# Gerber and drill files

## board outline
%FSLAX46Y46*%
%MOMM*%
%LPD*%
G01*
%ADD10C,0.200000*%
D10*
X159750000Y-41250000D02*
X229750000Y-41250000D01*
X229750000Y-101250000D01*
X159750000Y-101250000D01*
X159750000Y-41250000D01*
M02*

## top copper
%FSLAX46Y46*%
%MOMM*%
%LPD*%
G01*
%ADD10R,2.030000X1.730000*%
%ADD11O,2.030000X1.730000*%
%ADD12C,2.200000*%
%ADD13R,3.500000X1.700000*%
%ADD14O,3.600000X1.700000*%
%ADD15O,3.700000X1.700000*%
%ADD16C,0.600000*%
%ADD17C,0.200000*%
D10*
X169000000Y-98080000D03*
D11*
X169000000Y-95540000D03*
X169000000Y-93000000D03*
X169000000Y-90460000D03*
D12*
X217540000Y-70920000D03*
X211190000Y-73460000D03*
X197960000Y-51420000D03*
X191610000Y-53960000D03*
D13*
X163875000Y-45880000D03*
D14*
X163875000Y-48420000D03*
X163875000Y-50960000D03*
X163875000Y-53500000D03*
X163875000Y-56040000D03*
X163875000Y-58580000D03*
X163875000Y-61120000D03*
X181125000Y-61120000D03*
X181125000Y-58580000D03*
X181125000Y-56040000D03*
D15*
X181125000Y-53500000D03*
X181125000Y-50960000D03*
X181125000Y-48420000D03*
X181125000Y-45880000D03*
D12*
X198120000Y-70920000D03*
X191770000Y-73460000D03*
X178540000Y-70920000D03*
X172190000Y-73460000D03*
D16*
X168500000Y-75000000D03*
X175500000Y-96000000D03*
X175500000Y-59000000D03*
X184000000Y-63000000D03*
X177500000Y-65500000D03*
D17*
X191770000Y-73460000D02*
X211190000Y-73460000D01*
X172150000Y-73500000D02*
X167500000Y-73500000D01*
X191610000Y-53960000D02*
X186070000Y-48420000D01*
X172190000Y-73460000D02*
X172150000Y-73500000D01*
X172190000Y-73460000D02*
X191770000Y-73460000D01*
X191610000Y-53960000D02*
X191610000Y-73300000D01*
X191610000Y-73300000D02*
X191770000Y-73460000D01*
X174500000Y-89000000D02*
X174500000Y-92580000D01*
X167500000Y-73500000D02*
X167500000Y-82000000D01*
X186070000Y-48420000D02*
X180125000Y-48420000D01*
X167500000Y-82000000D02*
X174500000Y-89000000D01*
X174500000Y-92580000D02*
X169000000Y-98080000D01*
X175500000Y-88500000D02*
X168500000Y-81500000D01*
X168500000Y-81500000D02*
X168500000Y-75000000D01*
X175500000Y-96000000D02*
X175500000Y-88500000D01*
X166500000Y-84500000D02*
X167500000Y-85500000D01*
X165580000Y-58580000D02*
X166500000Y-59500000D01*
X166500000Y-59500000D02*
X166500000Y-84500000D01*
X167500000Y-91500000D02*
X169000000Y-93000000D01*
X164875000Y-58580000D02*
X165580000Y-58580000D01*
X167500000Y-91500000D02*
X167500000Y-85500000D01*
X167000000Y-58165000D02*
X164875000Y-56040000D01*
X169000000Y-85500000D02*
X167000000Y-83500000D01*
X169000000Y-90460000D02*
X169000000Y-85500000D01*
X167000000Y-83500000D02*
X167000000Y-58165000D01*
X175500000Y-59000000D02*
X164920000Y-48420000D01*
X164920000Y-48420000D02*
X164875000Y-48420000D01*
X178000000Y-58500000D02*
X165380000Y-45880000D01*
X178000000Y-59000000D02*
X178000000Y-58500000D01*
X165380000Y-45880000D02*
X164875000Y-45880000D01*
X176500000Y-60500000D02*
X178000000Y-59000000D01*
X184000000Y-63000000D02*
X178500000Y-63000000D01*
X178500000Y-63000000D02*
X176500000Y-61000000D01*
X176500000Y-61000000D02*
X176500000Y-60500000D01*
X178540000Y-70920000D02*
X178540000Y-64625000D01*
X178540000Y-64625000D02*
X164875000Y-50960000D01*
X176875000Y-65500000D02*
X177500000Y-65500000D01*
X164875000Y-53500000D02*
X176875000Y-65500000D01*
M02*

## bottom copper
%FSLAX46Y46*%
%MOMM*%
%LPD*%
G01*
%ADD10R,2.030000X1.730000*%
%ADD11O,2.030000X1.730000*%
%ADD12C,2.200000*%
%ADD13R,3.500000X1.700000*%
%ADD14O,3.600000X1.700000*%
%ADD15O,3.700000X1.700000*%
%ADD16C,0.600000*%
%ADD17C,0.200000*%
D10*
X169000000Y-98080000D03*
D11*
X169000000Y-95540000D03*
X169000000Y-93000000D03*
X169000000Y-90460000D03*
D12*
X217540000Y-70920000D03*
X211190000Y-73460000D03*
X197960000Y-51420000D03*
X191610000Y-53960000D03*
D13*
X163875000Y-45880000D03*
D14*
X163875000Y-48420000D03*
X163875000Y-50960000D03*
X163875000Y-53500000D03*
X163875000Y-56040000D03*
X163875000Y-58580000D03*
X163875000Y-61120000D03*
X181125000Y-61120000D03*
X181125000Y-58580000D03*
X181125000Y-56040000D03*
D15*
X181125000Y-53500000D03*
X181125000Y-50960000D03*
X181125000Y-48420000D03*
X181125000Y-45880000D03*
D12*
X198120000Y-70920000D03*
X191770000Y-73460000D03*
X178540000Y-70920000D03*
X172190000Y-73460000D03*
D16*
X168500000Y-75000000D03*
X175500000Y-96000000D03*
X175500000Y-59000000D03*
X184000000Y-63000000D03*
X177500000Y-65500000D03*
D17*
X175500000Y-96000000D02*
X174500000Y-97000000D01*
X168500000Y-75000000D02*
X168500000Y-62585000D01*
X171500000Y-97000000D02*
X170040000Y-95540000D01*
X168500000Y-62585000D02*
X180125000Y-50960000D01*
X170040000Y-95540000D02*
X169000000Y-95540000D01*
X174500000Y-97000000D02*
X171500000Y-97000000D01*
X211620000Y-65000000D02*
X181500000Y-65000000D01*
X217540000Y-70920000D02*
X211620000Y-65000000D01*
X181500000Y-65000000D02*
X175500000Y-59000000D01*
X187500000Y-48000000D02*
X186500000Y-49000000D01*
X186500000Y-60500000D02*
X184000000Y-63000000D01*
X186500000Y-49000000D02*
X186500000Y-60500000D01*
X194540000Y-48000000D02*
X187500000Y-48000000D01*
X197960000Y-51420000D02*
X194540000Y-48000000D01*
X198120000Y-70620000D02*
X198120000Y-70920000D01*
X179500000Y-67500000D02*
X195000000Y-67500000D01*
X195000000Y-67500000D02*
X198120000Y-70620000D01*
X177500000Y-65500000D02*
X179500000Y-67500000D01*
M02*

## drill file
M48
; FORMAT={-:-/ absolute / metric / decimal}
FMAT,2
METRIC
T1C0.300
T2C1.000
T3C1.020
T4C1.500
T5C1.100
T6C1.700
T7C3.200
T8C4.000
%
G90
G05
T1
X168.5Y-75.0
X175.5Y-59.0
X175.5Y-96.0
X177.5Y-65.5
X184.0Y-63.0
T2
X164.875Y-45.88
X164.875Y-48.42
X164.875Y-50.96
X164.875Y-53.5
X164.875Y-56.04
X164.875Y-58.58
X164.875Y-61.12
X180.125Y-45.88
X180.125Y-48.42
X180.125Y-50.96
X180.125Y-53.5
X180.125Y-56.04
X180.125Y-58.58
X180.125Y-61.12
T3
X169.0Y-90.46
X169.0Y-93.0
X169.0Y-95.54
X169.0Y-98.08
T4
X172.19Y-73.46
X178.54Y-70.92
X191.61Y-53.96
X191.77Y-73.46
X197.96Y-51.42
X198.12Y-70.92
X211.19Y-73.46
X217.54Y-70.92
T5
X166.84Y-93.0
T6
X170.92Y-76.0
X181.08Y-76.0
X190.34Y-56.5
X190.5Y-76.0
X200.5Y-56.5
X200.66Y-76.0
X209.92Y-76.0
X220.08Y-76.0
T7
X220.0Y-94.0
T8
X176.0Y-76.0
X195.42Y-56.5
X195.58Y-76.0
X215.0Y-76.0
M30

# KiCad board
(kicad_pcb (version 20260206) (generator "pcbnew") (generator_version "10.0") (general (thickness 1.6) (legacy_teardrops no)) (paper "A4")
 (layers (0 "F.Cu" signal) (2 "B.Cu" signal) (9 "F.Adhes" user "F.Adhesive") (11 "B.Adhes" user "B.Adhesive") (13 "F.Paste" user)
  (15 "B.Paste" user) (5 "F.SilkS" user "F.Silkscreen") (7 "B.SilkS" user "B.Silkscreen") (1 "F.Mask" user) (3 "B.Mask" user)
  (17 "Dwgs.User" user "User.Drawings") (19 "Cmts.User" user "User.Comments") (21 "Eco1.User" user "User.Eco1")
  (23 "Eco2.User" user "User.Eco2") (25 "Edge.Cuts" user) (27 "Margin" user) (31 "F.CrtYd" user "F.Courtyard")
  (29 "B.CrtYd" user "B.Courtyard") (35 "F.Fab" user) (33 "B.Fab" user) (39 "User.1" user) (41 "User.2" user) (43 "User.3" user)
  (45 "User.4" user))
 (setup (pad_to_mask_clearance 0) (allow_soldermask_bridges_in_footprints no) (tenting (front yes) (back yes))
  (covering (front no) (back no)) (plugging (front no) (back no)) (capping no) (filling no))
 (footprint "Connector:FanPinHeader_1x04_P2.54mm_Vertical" (layer "F.Cu") (at 169 98.08 90)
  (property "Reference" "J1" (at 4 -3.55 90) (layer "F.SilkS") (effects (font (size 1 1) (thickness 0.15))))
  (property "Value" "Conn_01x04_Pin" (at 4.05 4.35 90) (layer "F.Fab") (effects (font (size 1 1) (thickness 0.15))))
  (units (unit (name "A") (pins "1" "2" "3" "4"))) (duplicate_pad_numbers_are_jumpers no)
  (pad "" np_thru_hole circle (at 5.08 -2.16 180) (size 1.1 1.1) (drill 1.1) (layers "*.Cu" "*.Mask"))
  (pad "1" thru_hole rect (at 0 0 180) (size 2.03 1.73) (drill 1.02) (layers "*.Cu" "*.Mask") (remove_unused_layers no)
   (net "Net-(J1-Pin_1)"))
  (pad "2" thru_hole oval (at 2.54 0 180) (size 2.03 1.73) (drill 1.02) (layers "*.Cu" "*.Mask") (remove_unused_layers no)
   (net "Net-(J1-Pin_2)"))
  (pad "3" thru_hole oval (at 5.08 0 180) (size 2.03 1.73) (drill 1.02) (layers "*.Cu" "*.Mask") (remove_unused_layers no)
   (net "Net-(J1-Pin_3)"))
  (pad "4" thru_hole oval (at 7.62 0 180) (size 2.03 1.73) (drill 1.02) (layers "*.Cu" "*.Mask") (remove_unused_layers no)
   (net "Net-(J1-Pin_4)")))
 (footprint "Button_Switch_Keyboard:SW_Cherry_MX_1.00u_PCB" (layer "F.Cu") (at 217.54 70.92)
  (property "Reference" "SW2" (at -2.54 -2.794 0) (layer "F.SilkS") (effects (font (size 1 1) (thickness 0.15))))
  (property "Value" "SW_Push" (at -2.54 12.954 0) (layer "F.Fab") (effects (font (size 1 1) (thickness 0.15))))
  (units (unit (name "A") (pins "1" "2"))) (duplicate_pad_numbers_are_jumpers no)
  (pad "" np_thru_hole circle (at -7.62 5.08) (size 1.7 1.7) (drill 1.7) (layers "*.Cu" "*.Mask"))
  (pad "" np_thru_hole circle (at -2.54 5.08) (size 4 4) (drill 4) (layers "*.Cu" "*.Mask"))
  (pad "" np_thru_hole circle (at 2.54 5.08) (size 1.7 1.7) (drill 1.7) (layers "*.Cu" "*.Mask"))
  (pad "1" thru_hole circle (at 0 0) (size 2.2 2.2) (drill 1.5) (layers "*.Cu" "*.Mask") (remove_unused_layers no)
   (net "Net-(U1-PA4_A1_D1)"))
  (pad "2" thru_hole circle (at -6.35 2.54) (size 2.2 2.2) (drill 1.5) (layers "*.Cu" "*.Mask") (remove_unused_layers no)
   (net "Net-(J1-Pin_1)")))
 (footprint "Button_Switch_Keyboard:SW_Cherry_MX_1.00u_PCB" (layer "F.Cu") (at 197.96 51.42)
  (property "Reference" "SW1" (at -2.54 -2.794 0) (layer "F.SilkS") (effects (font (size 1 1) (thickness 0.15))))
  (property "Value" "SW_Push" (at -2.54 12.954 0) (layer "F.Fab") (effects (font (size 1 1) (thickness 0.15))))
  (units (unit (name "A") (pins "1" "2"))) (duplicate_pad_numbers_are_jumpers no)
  (pad "" np_thru_hole circle (at -7.62 5.08) (size 1.7 1.7) (drill 1.7) (layers "*.Cu" "*.Mask"))
  (pad "" np_thru_hole circle (at -2.54 5.08) (size 4 4) (drill 4) (layers "*.Cu" "*.Mask"))
  (pad "" np_thru_hole circle (at 2.54 5.08) (size 1.7 1.7) (drill 1.7) (layers "*.Cu" "*.Mask"))
  (pad "1" thru_hole circle (at 0 0) (size 2.2 2.2) (drill 1.5) (layers "*.Cu" "*.Mask") (remove_unused_layers no)
   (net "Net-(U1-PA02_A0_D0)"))
  (pad "2" thru_hole circle (at -6.35 2.54) (size 2.2 2.2) (drill 1.5) (layers "*.Cu" "*.Mask") (remove_unused_layers no)
   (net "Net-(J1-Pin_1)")))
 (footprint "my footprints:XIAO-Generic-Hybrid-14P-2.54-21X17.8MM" (layer "F.Cu") (at 172.5 53.5)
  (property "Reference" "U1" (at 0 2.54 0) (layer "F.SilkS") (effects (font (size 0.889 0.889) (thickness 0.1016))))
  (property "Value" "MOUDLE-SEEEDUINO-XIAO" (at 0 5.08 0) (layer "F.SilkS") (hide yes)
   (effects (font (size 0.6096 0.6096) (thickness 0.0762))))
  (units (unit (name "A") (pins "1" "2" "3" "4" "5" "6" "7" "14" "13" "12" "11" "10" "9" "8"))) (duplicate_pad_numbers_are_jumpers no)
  (pad "1" thru_hole rect (at -7.625 -7.62) (size 3.5 1.7) (drill 1 (offset -1 0)) (layers "*.Cu" "*.Mask") (remove_unused_layers no)
   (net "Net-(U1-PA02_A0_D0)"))
  (pad "2" thru_hole oval (at -7.625 -5.08) (size 3.6 1.7) (drill 1 (offset -1 0)) (layers "*.Cu" "*.Mask") (remove_unused_layers no)
   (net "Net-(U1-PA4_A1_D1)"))
  (pad "3" thru_hole oval (at -7.625 -2.54) (size 3.6 1.7) (drill 1 (offset -1 0)) (layers "*.Cu" "*.Mask") (remove_unused_layers no)
   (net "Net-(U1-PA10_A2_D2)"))
  (pad "4" thru_hole oval (at -7.625 0) (size 3.6 1.7) (drill 1 (offset -1 0)) (layers "*.Cu" "*.Mask") (remove_unused_layers no)
   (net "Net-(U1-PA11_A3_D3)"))
  (pad "5" thru_hole oval (at -7.625 2.54) (size 3.6 1.7) (drill 1 (offset -1 0)) (layers "*.Cu" "*.Mask") (remove_unused_layers no)
   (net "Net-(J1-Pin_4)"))
  (pad "6" thru_hole oval (at -7.625 5.08 180) (size 3.6 1.7) (drill 1 (offset 1 0)) (layers "*.Cu" "*.Mask") (remove_unused_layers no)
   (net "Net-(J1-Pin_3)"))
  (pad "7" thru_hole oval (at -7.625 7.62) (size 3.6 1.7) (drill 1 (offset -1 0)) (layers "*.Cu" "*.Mask") (remove_unused_layers no)
   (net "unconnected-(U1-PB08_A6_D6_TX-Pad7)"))
  (pad "8" thru_hole oval (at 7.625 7.62) (size 3.6 1.7) (drill 1 (offset 1 0)) (layers "*.Cu" "*.Mask") (remove_unused_layers no)
   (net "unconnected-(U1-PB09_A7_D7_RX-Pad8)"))
  (pad "9" thru_hole oval (at 7.625 5.08) (size 3.6 1.7) (drill 1 (offset 1 0)) (layers "*.Cu" "*.Mask") (remove_unused_layers no)
   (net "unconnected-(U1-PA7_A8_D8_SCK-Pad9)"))
  (pad "10" thru_hole oval (at 7.625 2.54) (size 3.6 1.7) (drill 1 (offset 1 0)) (layers "*.Cu" "*.Mask") (remove_unused_layers no)
   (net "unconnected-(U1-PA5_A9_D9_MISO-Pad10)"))
  (pad "11" thru_hole oval (at 7.625 0) (size 3.7 1.7) (drill 1 (offset 1 0)) (layers "*.Cu" "*.Mask") (remove_unused_layers no)
   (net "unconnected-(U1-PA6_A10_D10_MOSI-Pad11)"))
  (pad "12" thru_hole oval (at 7.625 -2.54) (size 3.7 1.7) (drill 1 (offset 1 0)) (layers "*.Cu" "*.Mask") (remove_unused_layers no)
   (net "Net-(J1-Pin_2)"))
  (pad "13" thru_hole oval (at 7.625 -5.08) (size 3.7 1.7) (drill 1 (offset 1 0)) (layers "*.Cu" "*.Mask") (remove_unused_layers no)
   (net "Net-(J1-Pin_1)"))
  (pad "14" thru_hole oval (at 7.625 -7.62) (size 3.7 1.7) (drill 1 (offset 1 0)) (layers "*.Cu" "*.Mask") (remove_unused_layers no)
   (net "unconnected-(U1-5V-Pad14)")))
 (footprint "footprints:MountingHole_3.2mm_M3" (layer "F.Cu") (at 220 94)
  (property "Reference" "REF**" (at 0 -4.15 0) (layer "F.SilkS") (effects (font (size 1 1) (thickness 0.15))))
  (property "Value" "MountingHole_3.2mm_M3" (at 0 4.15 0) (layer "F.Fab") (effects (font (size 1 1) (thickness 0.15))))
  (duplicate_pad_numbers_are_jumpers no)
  (pad "" np_thru_hole circle (at 0 0) (size 3.2 3.2) (drill 3.2) (layers "*.Cu" "*.Mask")))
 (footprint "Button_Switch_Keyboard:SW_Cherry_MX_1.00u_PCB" (layer "F.Cu") (at 198.12 70.92)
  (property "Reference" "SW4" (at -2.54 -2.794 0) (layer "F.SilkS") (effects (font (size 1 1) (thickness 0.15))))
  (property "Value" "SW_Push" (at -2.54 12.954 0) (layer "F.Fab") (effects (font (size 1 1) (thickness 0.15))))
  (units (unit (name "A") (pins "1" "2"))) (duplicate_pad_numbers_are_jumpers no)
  (pad "" np_thru_hole circle (at -7.62 5.08) (size 1.7 1.7) (drill 1.7) (layers "*.Cu" "*.Mask"))
  (pad "" np_thru_hole circle (at -2.54 5.08) (size 4 4) (drill 4) (layers "*.Cu" "*.Mask"))
  (pad "" np_thru_hole circle (at 2.54 5.08) (size 1.7 1.7) (drill 1.7) (layers "*.Cu" "*.Mask"))
  (pad "1" thru_hole circle (at 0 0) (size 2.2 2.2) (drill 1.5) (layers "*.Cu" "*.Mask") (remove_unused_layers no)
   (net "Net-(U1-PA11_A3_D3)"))
  (pad "2" thru_hole circle (at -6.35 2.54) (size 2.2 2.2) (drill 1.5) (layers "*.Cu" "*.Mask") (remove_unused_layers no)
   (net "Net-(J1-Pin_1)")))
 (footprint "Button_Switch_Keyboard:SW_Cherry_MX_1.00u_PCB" (layer "F.Cu") (at 178.54 70.92)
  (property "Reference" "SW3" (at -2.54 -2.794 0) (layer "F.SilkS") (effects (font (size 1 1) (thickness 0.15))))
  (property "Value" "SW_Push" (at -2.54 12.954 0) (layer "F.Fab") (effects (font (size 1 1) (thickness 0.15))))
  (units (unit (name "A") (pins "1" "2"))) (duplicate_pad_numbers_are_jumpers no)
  (pad "" np_thru_hole circle (at -7.62 5.08) (size 1.7 1.7) (drill 1.7) (layers "*.Cu" "*.Mask"))
  (pad "" np_thru_hole circle (at -2.54 5.08) (size 4 4) (drill 4) (layers "*.Cu" "*.Mask"))
  (pad "" np_thru_hole circle (at 2.54 5.08) (size 1.7 1.7) (drill 1.7) (layers "*.Cu" "*.Mask"))
  (pad "1" thru_hole circle (at 0 0) (size 2.2 2.2) (drill 1.5) (layers "*.Cu" "*.Mask") (remove_unused_layers no)
   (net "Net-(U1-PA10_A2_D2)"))
  (pad "2" thru_hole circle (at -6.35 2.54) (size 2.2 2.2) (drill 1.5) (layers "*.Cu" "*.Mask") (remove_unused_layers no)
   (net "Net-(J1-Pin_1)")))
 (gr_rect (start 159.75 41.25) (end 229.75 101.25) (stroke (width 0.2) (type solid)) (fill no) (layer "Edge.Cuts"))
 (segment (start 191.77 73.46) (end 211.19 73.46) (width 0.2) (layer "F.Cu") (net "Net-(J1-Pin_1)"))
 (segment (start 172.15 73.5) (end 167.5 73.5) (width 0.2) (layer "F.Cu") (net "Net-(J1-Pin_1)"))
 (segment (start 191.61 53.96) (end 186.07 48.42) (width 0.2) (layer "F.Cu") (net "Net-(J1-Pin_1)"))
 (segment (start 172.19 73.46) (end 172.15 73.5) (width 0.2) (layer "F.Cu") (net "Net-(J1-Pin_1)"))
 (segment (start 172.19 73.46) (end 191.77 73.46) (width 0.2) (layer "F.Cu") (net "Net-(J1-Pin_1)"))
 (segment (start 191.61 53.96) (end 191.61 73.3) (width 0.2) (layer "F.Cu") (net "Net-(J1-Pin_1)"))
 (segment (start 191.61 73.3) (end 191.77 73.46) (width 0.2) (layer "F.Cu") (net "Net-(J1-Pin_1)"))
 (segment (start 174.5 89) (end 174.5 92.58) (width 0.2) (layer "F.Cu") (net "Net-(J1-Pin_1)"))
 (segment (start 167.5 73.5) (end 167.5 82) (width 0.2) (layer "F.Cu") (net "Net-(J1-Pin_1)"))
 (segment (start 186.07 48.42) (end 180.125 48.42) (width 0.2) (layer "F.Cu") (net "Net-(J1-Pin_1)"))
 (segment (start 167.5 82) (end 174.5 89) (width 0.2) (layer "F.Cu") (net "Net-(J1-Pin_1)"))
 (segment (start 174.5 92.58) (end 169 98.08) (width 0.2) (layer "F.Cu") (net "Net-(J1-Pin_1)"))
 (segment (start 175.5 88.5) (end 168.5 81.5) (width 0.2) (layer "F.Cu") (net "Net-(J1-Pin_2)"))
 (segment (start 168.5 81.5) (end 168.5 75) (width 0.2) (layer "F.Cu") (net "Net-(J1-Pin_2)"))
 (segment (start 175.5 96) (end 175.5 88.5) (width 0.2) (layer "F.Cu") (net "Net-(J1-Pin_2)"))
 (via (at 168.5 75) (size 0.6) (drill 0.3) (layers "F.Cu" "B.Cu") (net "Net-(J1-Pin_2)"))
 (via (at 175.5 96) (size 0.6) (drill 0.3) (layers "F.Cu" "B.Cu") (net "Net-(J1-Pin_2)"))
 (segment (start 175.5 96) (end 174.5 97) (width 0.2) (layer "B.Cu") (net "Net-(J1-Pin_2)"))
 (segment (start 168.5 75) (end 168.5 62.585) (width 0.2) (layer "B.Cu") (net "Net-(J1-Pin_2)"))
 (segment (start 171.5 97) (end 170.04 95.54) (width 0.2) (layer "B.Cu") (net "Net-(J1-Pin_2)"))
 (segment (start 168.5 62.585) (end 180.125 50.96) (width 0.2) (layer "B.Cu") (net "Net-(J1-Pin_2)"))
 (segment (start 170.04 95.54) (end 169 95.54) (width 0.2) (layer "B.Cu") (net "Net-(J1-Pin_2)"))
 (segment (start 174.5 97) (end 171.5 97) (width 0.2) (layer "B.Cu") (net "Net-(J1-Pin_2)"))
 (segment (start 166.5 84.5) (end 167.5 85.5) (width 0.2) (layer "F.Cu") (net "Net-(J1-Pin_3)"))
 (segment (start 165.58 58.58) (end 166.5 59.5) (width 0.2) (layer "F.Cu") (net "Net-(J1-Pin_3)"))
 (segment (start 166.5 59.5) (end 166.5 84.5) (width 0.2) (layer "F.Cu") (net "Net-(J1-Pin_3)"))
 (segment (start 167.5 91.5) (end 169 93) (width 0.2) (layer "F.Cu") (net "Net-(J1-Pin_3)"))
 (segment (start 164.875 58.58) (end 165.58 58.58) (width 0.2) (layer "F.Cu") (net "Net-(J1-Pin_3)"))
 (segment (start 167.5 91.5) (end 167.5 85.5) (width 0.2) (layer "F.Cu") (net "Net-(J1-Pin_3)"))
 (segment (start 167 58.165) (end 164.875 56.04) (width 0.2) (layer "F.Cu") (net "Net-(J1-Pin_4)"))
 (segment (start 169 85.5) (end 167 83.5) (width 0.2) (layer "F.Cu") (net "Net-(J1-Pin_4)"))
 (segment (start 169 90.46) (end 169 85.5) (width 0.2) (layer "F.Cu") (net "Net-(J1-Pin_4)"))
 (segment (start 167 83.5) (end 167 58.165) (width 0.2) (layer "F.Cu") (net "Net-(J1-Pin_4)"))
 (segment (start 175.5 59) (end 164.92 48.42) (width 0.2) (layer "F.Cu") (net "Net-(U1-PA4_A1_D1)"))
 (segment (start 164.92 48.42) (end 164.875 48.42) (width 0.2) (layer "F.Cu") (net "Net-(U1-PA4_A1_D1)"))
 (via (at 175.5 59) (size 0.6) (drill 0.3) (layers "F.Cu" "B.Cu") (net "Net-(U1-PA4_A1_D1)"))
 (segment (start 211.62 65) (end 181.5 65) (width 0.2) (layer "B.Cu") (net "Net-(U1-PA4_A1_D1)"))
 (segment (start 217.54 70.92) (end 211.62 65) (width 0.2) (layer "B.Cu") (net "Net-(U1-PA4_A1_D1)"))
 (segment (start 181.5 65) (end 175.5 59) (width 0.2) (layer "B.Cu") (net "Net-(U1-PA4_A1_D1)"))
 (segment (start 178 58.5) (end 165.38 45.88) (width 0.2) (layer "F.Cu") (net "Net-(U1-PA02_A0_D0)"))
 (segment (start 178 59) (end 178 58.5) (width 0.2) (layer "F.Cu") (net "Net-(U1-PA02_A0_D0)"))
 (segment (start 165.38 45.88) (end 164.875 45.88) (width 0.2) (layer "F.Cu") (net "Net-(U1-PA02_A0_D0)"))
 (segment (start 176.5 60.5) (end 178 59) (width 0.2) (layer "F.Cu") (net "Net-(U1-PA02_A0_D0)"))
 (segment (start 184 63) (end 178.5 63) (width 0.2) (layer "F.Cu") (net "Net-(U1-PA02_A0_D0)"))
 (segment (start 178.5 63) (end 176.5 61) (width 0.2) (layer "F.Cu") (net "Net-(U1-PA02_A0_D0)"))
 (segment (start 176.5 61) (end 176.5 60.5) (width 0.2) (layer "F.Cu") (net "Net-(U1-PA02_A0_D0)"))
 (via (at 184 63) (size 0.6) (drill 0.3) (layers "F.Cu" "B.Cu") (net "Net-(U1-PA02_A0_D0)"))
 (segment (start 187.5 48) (end 186.5 49) (width 0.2) (layer "B.Cu") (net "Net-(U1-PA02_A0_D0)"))
 (segment (start 186.5 60.5) (end 184 63) (width 0.2) (layer "B.Cu") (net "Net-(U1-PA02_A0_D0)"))
 (segment (start 186.5 49) (end 186.5 60.5) (width 0.2) (layer "B.Cu") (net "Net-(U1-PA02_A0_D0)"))
 (segment (start 194.54 48) (end 187.5 48) (width 0.2) (layer "B.Cu") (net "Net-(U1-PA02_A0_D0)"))
 (segment (start 197.96 51.42) (end 194.54 48) (width 0.2) (layer "B.Cu") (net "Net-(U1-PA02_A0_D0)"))
 (segment (start 178.54 70.92) (end 178.54 64.625) (width 0.2) (layer "F.Cu") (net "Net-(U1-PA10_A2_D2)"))
 (segment (start 178.54 64.625) (end 164.875 50.96) (width 0.2) (layer "F.Cu") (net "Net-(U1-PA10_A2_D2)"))
 (segment (start 176.875 65.5) (end 177.5 65.5) (width 0.2) (layer "F.Cu") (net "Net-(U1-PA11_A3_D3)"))
 (segment (start 164.875 53.5) (end 176.875 65.5) (width 0.2) (layer "F.Cu") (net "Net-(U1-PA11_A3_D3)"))
 (via (at 177.5 65.5) (size 0.6) (drill 0.3) (layers "F.Cu" "B.Cu") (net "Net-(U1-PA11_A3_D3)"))
 (segment (start 198.12 70.62) (end 198.12 70.92) (width 0.2) (layer "B.Cu") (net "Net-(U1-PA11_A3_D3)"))
 (segment (start 179.5 67.5) (end 195 67.5) (width 0.2) (layer "B.Cu") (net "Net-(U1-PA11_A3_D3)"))
 (segment (start 195 67.5) (end 198.12 70.62) (width 0.2) (layer "B.Cu") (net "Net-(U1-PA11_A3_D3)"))
 (segment (start 177.5 65.5) (end 179.5 67.5) (width 0.2) (layer "B.Cu") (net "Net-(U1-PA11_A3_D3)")))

